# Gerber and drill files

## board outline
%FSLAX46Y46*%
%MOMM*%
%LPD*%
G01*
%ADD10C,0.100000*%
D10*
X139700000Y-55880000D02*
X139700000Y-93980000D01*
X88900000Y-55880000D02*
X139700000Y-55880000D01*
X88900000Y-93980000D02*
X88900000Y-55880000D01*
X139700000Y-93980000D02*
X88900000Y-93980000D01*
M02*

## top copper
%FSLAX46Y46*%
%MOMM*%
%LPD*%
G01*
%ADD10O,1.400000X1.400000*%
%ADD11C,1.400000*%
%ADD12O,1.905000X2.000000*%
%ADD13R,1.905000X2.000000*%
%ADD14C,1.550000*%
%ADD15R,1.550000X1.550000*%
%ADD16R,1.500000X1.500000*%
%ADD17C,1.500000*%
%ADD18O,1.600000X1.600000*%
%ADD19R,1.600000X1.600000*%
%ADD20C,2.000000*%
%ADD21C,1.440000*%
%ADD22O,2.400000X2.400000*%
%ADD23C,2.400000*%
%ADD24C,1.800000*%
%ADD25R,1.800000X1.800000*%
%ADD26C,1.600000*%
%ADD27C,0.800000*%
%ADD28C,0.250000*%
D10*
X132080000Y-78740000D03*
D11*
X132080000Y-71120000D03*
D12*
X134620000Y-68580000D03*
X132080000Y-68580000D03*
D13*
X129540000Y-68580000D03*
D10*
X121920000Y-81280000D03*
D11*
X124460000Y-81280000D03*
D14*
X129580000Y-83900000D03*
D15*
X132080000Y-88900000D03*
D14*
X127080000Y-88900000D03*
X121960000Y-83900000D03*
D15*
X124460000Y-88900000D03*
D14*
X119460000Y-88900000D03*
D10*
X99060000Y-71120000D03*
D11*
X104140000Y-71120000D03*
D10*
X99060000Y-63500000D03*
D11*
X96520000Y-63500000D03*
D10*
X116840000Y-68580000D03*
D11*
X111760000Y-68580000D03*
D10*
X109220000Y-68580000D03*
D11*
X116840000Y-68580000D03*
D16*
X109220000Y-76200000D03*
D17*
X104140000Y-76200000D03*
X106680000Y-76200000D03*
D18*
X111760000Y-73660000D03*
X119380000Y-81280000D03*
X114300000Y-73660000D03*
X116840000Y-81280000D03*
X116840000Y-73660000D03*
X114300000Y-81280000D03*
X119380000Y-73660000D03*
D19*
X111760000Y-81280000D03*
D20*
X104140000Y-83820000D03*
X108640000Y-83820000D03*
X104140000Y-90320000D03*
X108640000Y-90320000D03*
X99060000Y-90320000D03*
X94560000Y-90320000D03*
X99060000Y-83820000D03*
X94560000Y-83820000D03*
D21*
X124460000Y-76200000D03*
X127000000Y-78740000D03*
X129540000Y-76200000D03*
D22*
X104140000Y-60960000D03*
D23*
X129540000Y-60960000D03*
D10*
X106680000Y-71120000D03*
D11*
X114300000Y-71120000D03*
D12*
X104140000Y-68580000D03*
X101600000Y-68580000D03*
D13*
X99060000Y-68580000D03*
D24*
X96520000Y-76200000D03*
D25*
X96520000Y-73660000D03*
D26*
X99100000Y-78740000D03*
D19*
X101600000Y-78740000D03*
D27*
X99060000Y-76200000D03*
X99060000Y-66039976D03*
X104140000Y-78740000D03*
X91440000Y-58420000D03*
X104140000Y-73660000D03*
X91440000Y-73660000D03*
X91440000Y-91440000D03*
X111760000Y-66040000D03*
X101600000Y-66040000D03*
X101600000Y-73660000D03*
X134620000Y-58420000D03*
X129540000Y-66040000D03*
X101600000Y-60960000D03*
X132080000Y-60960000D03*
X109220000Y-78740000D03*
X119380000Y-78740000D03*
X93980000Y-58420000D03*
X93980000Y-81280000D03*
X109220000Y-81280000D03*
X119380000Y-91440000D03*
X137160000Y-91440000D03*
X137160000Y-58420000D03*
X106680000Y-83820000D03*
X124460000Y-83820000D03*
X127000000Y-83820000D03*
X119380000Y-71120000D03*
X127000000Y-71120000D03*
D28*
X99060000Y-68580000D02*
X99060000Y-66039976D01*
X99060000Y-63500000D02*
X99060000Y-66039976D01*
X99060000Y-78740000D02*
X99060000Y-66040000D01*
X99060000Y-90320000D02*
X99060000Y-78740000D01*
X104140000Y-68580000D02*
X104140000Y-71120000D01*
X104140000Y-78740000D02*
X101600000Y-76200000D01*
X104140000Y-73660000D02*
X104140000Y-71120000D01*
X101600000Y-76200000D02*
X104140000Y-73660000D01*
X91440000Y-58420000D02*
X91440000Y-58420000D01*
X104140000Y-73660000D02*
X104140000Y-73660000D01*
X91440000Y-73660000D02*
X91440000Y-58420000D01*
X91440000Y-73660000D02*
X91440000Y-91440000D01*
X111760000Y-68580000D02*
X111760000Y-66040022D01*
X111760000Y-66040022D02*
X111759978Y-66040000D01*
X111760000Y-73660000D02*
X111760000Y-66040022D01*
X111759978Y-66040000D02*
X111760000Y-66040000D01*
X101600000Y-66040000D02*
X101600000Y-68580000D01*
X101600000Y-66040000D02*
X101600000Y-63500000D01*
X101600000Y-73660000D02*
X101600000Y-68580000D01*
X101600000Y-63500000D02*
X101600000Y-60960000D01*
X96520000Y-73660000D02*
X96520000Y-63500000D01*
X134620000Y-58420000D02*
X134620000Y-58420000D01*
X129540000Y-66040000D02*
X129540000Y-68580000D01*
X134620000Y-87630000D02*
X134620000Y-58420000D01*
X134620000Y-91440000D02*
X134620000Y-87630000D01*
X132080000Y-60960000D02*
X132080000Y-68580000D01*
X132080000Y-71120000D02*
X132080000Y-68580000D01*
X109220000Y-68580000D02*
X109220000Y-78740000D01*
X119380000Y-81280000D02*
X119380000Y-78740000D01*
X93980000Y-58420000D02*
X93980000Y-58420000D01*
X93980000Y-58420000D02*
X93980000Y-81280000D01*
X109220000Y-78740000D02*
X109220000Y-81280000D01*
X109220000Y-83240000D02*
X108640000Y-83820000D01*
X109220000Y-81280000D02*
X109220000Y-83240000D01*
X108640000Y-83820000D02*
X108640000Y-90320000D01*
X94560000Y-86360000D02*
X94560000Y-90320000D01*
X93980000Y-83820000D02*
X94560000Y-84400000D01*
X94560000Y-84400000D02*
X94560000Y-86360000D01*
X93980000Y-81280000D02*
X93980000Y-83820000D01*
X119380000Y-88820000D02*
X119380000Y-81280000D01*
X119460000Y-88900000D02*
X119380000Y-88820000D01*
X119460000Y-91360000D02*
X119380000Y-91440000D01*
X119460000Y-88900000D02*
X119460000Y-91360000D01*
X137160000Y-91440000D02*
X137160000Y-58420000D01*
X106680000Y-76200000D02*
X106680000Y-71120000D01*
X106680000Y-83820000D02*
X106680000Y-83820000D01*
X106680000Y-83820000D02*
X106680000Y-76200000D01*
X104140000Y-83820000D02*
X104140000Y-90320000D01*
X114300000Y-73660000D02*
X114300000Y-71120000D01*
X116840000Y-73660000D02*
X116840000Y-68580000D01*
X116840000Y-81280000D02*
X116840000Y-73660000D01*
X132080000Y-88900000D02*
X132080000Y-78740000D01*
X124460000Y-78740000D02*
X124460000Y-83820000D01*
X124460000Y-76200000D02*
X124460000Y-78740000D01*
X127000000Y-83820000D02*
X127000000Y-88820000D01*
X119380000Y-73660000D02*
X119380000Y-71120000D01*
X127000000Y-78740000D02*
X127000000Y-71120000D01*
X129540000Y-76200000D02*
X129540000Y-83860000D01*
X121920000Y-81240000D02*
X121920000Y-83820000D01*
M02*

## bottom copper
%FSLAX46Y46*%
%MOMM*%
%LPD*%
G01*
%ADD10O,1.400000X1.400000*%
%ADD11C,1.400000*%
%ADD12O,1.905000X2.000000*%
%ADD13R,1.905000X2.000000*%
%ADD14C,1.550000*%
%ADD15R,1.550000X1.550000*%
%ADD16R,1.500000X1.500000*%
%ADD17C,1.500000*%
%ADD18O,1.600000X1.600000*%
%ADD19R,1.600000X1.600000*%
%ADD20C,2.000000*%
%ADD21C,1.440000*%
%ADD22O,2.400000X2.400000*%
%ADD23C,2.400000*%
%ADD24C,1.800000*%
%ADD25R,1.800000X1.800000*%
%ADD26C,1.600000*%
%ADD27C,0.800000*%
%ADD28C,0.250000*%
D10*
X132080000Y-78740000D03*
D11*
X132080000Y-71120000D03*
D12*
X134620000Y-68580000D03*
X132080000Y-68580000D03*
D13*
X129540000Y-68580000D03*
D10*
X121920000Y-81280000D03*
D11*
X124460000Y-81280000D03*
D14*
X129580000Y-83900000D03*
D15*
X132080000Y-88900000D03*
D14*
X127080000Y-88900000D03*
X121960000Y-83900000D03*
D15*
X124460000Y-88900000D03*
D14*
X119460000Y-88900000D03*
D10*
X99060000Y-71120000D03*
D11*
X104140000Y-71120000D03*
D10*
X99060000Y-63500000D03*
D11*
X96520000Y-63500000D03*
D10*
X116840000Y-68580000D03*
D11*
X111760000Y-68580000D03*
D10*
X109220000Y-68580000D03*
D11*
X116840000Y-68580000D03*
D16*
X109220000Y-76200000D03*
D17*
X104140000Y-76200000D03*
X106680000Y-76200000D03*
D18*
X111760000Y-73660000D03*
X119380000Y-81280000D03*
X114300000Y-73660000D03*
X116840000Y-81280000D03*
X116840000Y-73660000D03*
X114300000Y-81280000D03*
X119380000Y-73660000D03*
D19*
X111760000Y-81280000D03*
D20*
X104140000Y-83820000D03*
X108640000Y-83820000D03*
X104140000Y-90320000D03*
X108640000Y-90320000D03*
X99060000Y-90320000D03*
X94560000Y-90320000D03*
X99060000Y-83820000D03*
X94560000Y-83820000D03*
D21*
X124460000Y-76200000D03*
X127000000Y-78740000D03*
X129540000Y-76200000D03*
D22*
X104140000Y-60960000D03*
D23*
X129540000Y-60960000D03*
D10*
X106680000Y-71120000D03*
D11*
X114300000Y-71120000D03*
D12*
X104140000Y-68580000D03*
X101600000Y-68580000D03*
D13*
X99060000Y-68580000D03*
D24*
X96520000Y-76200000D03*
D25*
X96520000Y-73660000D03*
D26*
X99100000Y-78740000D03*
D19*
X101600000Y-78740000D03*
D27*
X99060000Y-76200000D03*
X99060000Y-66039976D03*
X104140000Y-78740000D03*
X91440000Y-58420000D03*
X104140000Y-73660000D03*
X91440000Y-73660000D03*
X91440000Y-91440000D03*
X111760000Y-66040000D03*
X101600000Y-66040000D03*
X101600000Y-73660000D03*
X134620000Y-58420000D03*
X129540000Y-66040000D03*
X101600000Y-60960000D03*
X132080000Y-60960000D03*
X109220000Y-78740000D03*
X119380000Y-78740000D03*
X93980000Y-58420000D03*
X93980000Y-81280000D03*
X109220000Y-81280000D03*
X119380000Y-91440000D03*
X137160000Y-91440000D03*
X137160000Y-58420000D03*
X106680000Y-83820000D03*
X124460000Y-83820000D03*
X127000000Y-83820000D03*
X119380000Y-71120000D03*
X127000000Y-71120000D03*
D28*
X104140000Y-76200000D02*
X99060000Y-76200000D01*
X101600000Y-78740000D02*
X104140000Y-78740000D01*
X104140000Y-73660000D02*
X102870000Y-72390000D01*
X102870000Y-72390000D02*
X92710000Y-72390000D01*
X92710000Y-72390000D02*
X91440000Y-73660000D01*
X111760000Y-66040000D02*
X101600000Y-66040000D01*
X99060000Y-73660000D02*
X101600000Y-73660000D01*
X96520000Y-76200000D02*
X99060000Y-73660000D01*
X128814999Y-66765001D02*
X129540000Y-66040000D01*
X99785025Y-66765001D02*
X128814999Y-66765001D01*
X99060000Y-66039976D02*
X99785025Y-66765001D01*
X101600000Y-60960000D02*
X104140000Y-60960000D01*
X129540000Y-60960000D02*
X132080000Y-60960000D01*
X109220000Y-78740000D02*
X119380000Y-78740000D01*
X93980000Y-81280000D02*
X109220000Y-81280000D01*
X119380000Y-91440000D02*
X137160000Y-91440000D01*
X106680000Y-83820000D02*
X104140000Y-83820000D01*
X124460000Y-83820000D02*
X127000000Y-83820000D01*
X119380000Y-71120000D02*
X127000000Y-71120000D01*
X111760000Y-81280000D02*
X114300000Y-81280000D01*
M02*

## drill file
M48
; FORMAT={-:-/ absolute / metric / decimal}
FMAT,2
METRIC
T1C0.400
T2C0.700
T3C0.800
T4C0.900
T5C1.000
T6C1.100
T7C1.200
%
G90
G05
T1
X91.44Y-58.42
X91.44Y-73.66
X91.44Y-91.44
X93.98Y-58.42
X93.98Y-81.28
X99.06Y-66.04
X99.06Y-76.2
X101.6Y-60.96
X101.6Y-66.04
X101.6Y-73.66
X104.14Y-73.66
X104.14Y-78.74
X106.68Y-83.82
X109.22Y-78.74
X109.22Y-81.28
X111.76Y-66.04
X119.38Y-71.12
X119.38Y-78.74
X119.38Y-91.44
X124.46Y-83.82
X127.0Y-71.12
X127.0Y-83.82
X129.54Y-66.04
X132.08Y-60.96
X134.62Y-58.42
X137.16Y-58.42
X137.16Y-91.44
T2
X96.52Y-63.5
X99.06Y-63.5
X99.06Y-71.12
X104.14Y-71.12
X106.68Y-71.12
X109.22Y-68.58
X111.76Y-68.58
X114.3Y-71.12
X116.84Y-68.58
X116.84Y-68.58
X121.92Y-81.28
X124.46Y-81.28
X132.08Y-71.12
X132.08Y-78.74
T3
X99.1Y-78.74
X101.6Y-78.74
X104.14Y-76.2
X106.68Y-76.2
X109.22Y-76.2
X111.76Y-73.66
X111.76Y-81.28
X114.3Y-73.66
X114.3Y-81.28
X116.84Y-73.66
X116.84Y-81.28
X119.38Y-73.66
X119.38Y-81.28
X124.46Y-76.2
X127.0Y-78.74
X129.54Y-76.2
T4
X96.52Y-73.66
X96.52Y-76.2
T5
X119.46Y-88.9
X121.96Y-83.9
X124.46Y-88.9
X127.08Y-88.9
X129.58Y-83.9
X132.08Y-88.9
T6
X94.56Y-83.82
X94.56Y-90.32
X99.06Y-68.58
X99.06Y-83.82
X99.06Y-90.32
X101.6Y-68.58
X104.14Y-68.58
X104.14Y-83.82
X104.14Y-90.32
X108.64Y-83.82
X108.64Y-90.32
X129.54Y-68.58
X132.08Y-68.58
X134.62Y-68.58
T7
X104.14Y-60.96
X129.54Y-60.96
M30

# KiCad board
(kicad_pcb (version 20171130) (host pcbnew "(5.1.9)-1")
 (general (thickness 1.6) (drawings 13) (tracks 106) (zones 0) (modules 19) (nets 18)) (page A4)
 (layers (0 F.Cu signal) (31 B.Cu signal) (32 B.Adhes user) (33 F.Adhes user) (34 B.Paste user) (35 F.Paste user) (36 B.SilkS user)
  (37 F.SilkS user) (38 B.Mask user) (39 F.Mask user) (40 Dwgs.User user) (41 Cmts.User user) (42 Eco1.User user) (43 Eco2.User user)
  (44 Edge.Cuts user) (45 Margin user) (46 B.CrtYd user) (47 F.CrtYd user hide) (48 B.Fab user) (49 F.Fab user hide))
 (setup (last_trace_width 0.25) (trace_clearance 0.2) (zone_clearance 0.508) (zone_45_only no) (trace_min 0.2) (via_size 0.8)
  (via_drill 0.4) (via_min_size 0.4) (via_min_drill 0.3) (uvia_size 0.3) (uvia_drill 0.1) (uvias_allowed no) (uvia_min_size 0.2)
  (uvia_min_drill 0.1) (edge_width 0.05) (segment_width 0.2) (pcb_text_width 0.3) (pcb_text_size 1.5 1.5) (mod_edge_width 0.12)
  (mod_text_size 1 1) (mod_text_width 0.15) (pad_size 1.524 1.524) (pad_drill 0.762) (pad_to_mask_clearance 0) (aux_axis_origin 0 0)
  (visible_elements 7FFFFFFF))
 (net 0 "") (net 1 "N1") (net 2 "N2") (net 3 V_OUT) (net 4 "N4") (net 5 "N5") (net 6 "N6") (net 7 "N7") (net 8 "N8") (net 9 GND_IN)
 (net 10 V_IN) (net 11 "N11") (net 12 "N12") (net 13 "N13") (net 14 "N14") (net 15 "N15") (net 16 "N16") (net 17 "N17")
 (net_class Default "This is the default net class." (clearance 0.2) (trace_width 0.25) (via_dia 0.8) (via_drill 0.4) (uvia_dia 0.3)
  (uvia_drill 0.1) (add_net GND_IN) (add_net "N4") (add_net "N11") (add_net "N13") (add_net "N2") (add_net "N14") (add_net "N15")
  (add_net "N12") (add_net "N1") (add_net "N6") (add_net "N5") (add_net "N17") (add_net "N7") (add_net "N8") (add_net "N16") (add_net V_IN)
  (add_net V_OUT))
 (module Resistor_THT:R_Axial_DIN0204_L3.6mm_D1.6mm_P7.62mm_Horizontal (layer F.Cu) (at 132.08 71.12 270)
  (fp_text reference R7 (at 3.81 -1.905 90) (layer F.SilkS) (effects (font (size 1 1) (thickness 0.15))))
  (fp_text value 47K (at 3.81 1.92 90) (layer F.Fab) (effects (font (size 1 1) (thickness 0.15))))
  (pad 2 thru_hole oval (at 7.62 0 270) (size 1.4 1.4) (drill 0.7) (layers *.Cu *.Mask) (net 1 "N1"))
  (pad 1 thru_hole circle (at 0 0 270) (size 1.4 1.4) (drill 0.7) (layers *.Cu *.Mask) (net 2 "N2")))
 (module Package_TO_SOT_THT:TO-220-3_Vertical (layer F.Cu) (at 129.54 68.58)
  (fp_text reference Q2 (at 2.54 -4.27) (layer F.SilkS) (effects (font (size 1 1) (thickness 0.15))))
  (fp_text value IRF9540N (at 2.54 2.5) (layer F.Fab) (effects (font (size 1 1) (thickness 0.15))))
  (pad 3 thru_hole oval (at 5.08 0) (size 1.905 2) (drill 1.1) (layers *.Cu *.Mask) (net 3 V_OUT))
  (pad 2 thru_hole oval (at 2.54 0) (size 1.905 2) (drill 1.1) (layers *.Cu *.Mask) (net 2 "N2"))
  (pad 1 thru_hole rect (at 0 0) (size 1.905 2) (drill 1.1) (layers *.Cu *.Mask) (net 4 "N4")))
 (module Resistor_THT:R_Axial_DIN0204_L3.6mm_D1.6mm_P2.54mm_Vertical (layer F.Cu) (at 124.46 81.28 180)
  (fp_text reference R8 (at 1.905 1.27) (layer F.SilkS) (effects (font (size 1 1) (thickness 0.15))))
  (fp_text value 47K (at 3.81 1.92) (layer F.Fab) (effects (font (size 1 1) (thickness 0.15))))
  (pad 2 thru_hole oval (at 2.54 0 180) (size 1.4 1.4) (drill 0.7) (layers *.Cu *.Mask) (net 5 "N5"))
  (pad 1 thru_hole circle (at 0 0 180) (size 1.4 1.4) (drill 0.7) (layers *.Cu *.Mask) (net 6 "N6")))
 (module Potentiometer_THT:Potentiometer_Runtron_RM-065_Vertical (layer F.Cu) (at 132.08 88.9 180)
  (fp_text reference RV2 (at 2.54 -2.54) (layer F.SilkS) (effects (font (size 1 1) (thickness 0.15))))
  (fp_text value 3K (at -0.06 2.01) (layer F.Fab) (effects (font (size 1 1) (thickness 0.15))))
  (pad 2 thru_hole circle (at 2.5 5 180) (size 1.55 1.55) (drill 1) (layers *.Cu *.Mask) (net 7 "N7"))
  (pad 1 thru_hole rect (at 0 0 180) (size 1.55 1.55) (drill 1) (layers *.Cu *.Mask) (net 1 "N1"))
  (pad 3 thru_hole circle (at 5 0 180) (size 1.55 1.55) (drill 1) (layers *.Cu *.Mask) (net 6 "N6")))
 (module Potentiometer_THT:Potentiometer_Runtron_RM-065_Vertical (layer F.Cu) (at 124.46 88.9 180)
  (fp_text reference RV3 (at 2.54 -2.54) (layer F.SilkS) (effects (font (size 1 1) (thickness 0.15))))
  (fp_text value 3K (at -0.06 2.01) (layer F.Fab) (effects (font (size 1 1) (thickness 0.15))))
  (pad 2 thru_hole circle (at 2.5 5 180) (size 1.55 1.55) (drill 1) (layers *.Cu *.Mask) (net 5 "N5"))
  (pad 1 thru_hole rect (at 0 0 180) (size 1.55 1.55) (drill 1) (layers *.Cu *.Mask) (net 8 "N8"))
  (pad 3 thru_hole circle (at 5 0 180) (size 1.55 1.55) (drill 1) (layers *.Cu *.Mask) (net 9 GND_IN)))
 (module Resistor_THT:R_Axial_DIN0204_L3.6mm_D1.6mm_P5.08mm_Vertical (layer F.Cu) (at 104.14 71.12 180)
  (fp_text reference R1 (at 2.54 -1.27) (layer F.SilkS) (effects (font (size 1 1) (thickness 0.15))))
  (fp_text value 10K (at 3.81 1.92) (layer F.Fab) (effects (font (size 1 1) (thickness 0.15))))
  (pad 2 thru_hole oval (at 5.08 0 180) (size 1.4 1.4) (drill 0.7) (layers *.Cu *.Mask) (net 4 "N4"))
  (pad 1 thru_hole circle (at 0 0 180) (size 1.4 1.4) (drill 0.7) (layers *.Cu *.Mask) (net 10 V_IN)))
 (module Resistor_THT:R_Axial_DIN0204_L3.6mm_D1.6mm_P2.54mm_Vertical (layer F.Cu) (at 96.52 63.5)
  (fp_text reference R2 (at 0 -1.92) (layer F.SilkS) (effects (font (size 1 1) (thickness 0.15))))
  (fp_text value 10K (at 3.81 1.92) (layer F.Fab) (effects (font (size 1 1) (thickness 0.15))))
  (pad 2 thru_hole oval (at 2.54 0) (size 1.4 1.4) (drill 0.7) (layers *.Cu *.Mask) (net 4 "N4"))
  (pad 1 thru_hole circle (at 0 0) (size 1.4 1.4) (drill 0.7) (layers *.Cu *.Mask) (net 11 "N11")))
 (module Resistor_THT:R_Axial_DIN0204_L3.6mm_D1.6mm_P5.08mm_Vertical (layer F.Cu) (at 111.76 68.58)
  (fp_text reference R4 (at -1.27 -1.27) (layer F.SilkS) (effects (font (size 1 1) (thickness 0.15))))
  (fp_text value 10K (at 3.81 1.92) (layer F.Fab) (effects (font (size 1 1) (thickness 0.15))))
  (pad 2 thru_hole oval (at 5.08 0) (size 1.4 1.4) (drill 0.7) (layers *.Cu *.Mask) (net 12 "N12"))
  (pad 1 thru_hole circle (at 0 0) (size 1.4 1.4) (drill 0.7) (layers *.Cu *.Mask) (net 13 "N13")))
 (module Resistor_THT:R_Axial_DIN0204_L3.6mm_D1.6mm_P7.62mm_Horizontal (layer F.Cu) (at 116.84 68.58 180)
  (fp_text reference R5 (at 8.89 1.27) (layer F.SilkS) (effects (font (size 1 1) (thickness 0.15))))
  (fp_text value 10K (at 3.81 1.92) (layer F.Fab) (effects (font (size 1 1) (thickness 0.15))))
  (pad 2 thru_hole oval (at 7.62 0 180) (size 1.4 1.4) (drill 0.7) (layers *.Cu *.Mask) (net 9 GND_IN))
  (pad 1 thru_hole circle (at 0 0 180) (size 1.4 1.4) (drill 0.7) (layers *.Cu *.Mask) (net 12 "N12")))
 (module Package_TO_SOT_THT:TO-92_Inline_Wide (layer F.Cu) (at 109.22 76.2 180)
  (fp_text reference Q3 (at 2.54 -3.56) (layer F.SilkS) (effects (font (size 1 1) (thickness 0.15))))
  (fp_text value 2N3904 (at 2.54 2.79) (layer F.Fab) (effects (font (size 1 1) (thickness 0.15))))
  (pad 1 thru_hole rect (at 0 0 180) (size 1.5 1.5) (drill 0.8) (layers *.Cu *.Mask) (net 9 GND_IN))
  (pad 3 thru_hole circle (at 5.08 0 180) (size 1.5 1.5) (drill 0.8) (layers *.Cu *.Mask) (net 4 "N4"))
  (pad 2 thru_hole circle (at 2.54 0 180) (size 1.5 1.5) (drill 0.8) (layers *.Cu *.Mask) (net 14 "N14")))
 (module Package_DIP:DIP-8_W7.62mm (layer F.Cu) (at 111.76 81.28 90)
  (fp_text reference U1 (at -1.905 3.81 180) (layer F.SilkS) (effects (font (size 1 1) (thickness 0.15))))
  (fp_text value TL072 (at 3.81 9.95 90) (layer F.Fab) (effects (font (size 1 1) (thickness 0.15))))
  (pad 8 thru_hole oval (at 7.62 0 90) (size 1.6 1.6) (drill 0.8) (layers *.Cu *.Mask) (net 13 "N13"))
  (pad 4 thru_hole oval (at 0 7.62 90) (size 1.6 1.6) (drill 0.8) (layers *.Cu *.Mask) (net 9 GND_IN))
  (pad 7 thru_hole oval (at 7.62 2.54 90) (size 1.6 1.6) (drill 0.8) (layers *.Cu *.Mask) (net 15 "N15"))
  (pad 3 thru_hole oval (at 0 5.08 90) (size 1.6 1.6) (drill 0.8) (layers *.Cu *.Mask) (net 12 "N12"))
  (pad 6 thru_hole oval (at 7.62 5.08 90) (size 1.6 1.6) (drill 0.8) (layers *.Cu *.Mask) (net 12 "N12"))
  (pad 2 thru_hole oval (at 0 2.54 90) (size 1.6 1.6) (drill 0.8) (layers *.Cu *.Mask) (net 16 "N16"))
  (pad 5 thru_hole oval (at 7.62 7.62 90) (size 1.6 1.6) (drill 0.8) (layers *.Cu *.Mask) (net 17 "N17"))
  (pad 1 thru_hole rect (at 0 0 90) (size 1.6 1.6) (drill 0.8) (layers *.Cu *.Mask) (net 16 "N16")))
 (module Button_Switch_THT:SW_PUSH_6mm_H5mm (layer F.Cu) (at 104.14 90.32 90)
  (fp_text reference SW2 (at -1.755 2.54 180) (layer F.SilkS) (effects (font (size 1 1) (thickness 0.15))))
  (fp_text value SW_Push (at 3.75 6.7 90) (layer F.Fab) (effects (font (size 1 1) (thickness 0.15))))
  (pad 1 thru_hole circle (at 6.5 0 180) (size 2 2) (drill 1.1) (layers *.Cu *.Mask) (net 14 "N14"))
  (pad 2 thru_hole circle (at 6.5 4.5 180) (size 2 2) (drill 1.1) (layers *.Cu *.Mask) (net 9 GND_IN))
  (pad 1 thru_hole circle (at 0 0 180) (size 2 2) (drill 1.1) (layers *.Cu *.Mask) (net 14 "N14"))
  (pad 2 thru_hole circle (at 0 4.5 180) (size 2 2) (drill 1.1) (layers *.Cu *.Mask) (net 9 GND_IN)))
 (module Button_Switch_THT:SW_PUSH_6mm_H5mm (layer F.Cu) (at 99.06 83.82 270)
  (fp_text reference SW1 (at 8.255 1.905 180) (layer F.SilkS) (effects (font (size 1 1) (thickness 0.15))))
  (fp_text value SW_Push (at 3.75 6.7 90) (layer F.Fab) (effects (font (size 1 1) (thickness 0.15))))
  (pad 1 thru_hole circle (at 6.5 0) (size 2 2) (drill 1.1) (layers *.Cu *.Mask) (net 4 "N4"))
  (pad 2 thru_hole circle (at 6.5 4.5) (size 2 2) (drill 1.1) (layers *.Cu *.Mask) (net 9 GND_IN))
  (pad 1 thru_hole circle (at 0 0) (size 2 2) (drill 1.1) (layers *.Cu *.Mask) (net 4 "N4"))
  (pad 2 thru_hole circle (at 0 4.5) (size 2 2) (drill 1.1) (layers *.Cu *.Mask) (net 9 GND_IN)))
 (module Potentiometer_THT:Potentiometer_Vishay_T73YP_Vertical (layer F.Cu) (at 124.46 76.2 270)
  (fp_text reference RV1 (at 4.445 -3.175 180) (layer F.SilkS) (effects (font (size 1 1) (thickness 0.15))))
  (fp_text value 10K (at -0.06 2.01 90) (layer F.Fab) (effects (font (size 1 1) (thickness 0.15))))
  (pad 1 thru_hole circle (at 0 0 270) (size 1.44 1.44) (drill 0.8) (layers *.Cu *.Mask) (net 6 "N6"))
  (pad 2 thru_hole circle (at 2.54 -2.54 270) (size 1.44 1.44) (drill 0.8) (layers *.Cu *.Mask) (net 17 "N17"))
  (pad 3 thru_hole circle (at 0 -5.08 270) (size 1.44 1.44) (drill 0.8) (layers *.Cu *.Mask) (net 7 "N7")))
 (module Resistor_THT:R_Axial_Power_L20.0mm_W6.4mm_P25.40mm (layer F.Cu) (at 129.54 60.96 180)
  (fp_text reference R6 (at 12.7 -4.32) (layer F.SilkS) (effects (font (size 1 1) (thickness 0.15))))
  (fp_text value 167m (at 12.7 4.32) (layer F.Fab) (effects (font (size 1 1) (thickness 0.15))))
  (pad 2 thru_hole oval (at 25.4 0 180) (size 2.4 2.4) (drill 1.2) (layers *.Cu *.Mask) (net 13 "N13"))
  (pad 1 thru_hole circle (at 0 0 180) (size 2.4 2.4) (drill 1.2) (layers *.Cu *.Mask) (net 2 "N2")))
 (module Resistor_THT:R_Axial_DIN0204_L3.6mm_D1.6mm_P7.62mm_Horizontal (layer F.Cu) (at 114.3 71.12 180)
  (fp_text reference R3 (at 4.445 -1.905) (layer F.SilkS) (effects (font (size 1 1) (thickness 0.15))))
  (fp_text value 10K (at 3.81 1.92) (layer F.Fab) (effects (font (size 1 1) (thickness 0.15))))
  (pad 2 thru_hole oval (at 7.62 0 180) (size 1.4 1.4) (drill 0.7) (layers *.Cu *.Mask) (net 14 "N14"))
  (pad 1 thru_hole circle (at 0 0 180) (size 1.4 1.4) (drill 0.7) (layers *.Cu *.Mask) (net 15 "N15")))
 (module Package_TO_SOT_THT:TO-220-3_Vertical (layer F.Cu) (at 99.06 68.58)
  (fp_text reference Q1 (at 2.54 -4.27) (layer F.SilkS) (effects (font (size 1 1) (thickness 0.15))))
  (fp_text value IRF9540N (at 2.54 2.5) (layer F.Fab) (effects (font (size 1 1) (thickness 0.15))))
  (pad 3 thru_hole oval (at 5.08 0) (size 1.905 2) (drill 1.1) (layers *.Cu *.Mask) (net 10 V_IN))
  (pad 2 thru_hole oval (at 2.54 0) (size 1.905 2) (drill 1.1) (layers *.Cu *.Mask) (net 13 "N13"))
  (pad 1 thru_hole rect (at 0 0) (size 1.905 2) (drill 1.1) (layers *.Cu *.Mask) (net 4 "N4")))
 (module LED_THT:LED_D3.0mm (layer F.Cu) (at 96.52 73.66 270)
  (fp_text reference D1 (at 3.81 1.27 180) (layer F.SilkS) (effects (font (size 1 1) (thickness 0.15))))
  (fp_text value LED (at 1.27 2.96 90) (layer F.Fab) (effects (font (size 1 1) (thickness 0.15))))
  (pad 2 thru_hole circle (at 2.54 0 270) (size 1.8 1.8) (drill 0.9) (layers *.Cu *.Mask) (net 13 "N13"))
  (pad 1 thru_hole rect (at 0 0 270) (size 1.8 1.8) (drill 0.9) (layers *.Cu *.Mask) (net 11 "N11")))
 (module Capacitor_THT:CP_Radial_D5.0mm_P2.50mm (layer F.Cu) (at 101.6 78.74 180)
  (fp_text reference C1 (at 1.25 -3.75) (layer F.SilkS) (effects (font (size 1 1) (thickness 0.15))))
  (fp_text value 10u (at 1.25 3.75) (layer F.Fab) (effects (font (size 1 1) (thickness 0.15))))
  (pad 2 thru_hole circle (at 2.5 0 180) (size 1.6 1.6) (drill 0.8) (layers *.Cu *.Mask) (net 4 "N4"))
  (pad 1 thru_hole rect (at 0 0 180) (size 1.6 1.6) (drill 0.8) (layers *.Cu *.Mask) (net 10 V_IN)))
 (gr_line (start 139.7 55.88) (end 139.7 93.98) (layer Edge.Cuts) (width 0.1))
 (gr_line (start 88.9 55.88) (end 139.7 55.88) (layer Edge.Cuts) (width 0.1))
 (gr_line (start 88.9 93.98) (end 88.9 55.88) (layer Edge.Cuts) (width 0.1))
 (gr_line (start 139.7 93.98) (end 88.9 93.98) (layer Edge.Cuts) (width 0.1))
 (via (at 99.06 76.2) (size 0.8) (drill 0.4) (layers F.Cu B.Cu) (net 4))
 (segment (start 104.14 76.2) (end 99.06 76.2) (width 0.25) (layer B.Cu) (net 4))
 (via (at 99.06 66.039976) (size 0.8) (drill 0.4) (layers F.Cu B.Cu) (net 4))
 (segment (start 99.06 68.58) (end 99.06 66.039976) (width 0.25) (layer F.Cu) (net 4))
 (segment (start 99.06 63.5) (end 99.06 66.039976) (width 0.25) (layer F.Cu) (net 4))
 (segment (start 99.06 78.74) (end 99.06 66.04) (width 0.25) (layer F.Cu) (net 4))
 (segment (start 99.06 90.32) (end 99.06 78.74) (width 0.25) (layer F.Cu) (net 4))
 (segment (start 104.14 68.58) (end 104.14 71.12) (width 0.25) (layer F.Cu) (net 10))
 (via (at 104.14 78.74) (size 0.8) (drill 0.4) (layers F.Cu B.Cu) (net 10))
 (segment (start 101.6 78.74) (end 104.14 78.74) (width 0.25) (layer B.Cu) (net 10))
 (segment (start 104.14 78.74) (end 101.6 76.2) (width 0.25) (layer F.Cu) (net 10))
 (segment (start 104.14 73.66) (end 104.14 71.12) (width 0.25) (layer F.Cu) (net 10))
 (segment (start 101.6 76.2) (end 104.14 73.66) (width 0.25) (layer F.Cu) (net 10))
 (segment (start 91.44 58.42) (end 91.44 58.42) (width 0.25) (layer F.Cu) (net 10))
 (via (at 91.44 58.42) (size 0.8) (drill 0.4) (layers F.Cu B.Cu) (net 10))
 (segment (start 104.14 73.66) (end 104.14 73.66) (width 0.25) (layer F.Cu) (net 10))
 (via (at 104.14 73.66) (size 0.8) (drill 0.4) (layers F.Cu B.Cu) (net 10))
 (segment (start 104.14 73.66) (end 102.87 72.39) (width 0.25) (layer B.Cu) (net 10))
 (segment (start 102.87 72.39) (end 92.71 72.39) (width 0.25) (layer B.Cu) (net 10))
 (via (at 91.44 73.66) (size 0.8) (drill 0.4) (layers F.Cu B.Cu) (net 10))
 (segment (start 92.71 72.39) (end 91.44 73.66) (width 0.25) (layer B.Cu) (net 10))
 (segment (start 91.44 73.66) (end 91.44 58.42) (width 0.25) (layer F.Cu) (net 10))
 (via (at 91.44 91.44) (size 0.8) (drill 0.4) (layers F.Cu B.Cu) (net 10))
 (segment (start 91.44 73.66) (end 91.44 91.44) (width 0.25) (layer F.Cu) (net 10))
 (segment (start 111.76 68.58) (end 111.76 66.040022) (width 0.25) (layer F.Cu) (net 13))
 (segment (start 111.76 66.040022) (end 111.759978 66.04) (width 0.25) (layer F.Cu) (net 13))
 (segment (start 111.76 73.66) (end 111.76 66.040022) (width 0.25) (layer F.Cu) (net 13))
 (via (at 111.76 66.04) (size 0.8) (drill 0.4) (layers F.Cu B.Cu) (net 13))
 (segment (start 111.759978 66.04) (end 111.76 66.04) (width 0.25) (layer F.Cu) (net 13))
 (via (at 101.6 66.04) (size 0.8) (drill 0.4) (layers F.Cu B.Cu) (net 13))
 (segment (start 111.76 66.04) (end 101.6 66.04) (width 0.25) (layer B.Cu) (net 13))
 (segment (start 101.6 66.04) (end 101.6 68.58) (width 0.25) (layer F.Cu) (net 13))
 (segment (start 101.6 66.04) (end 101.6 63.5) (width 0.25) (layer F.Cu) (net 13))
 (via (at 101.6 73.66) (size 0.8) (drill 0.4) (layers F.Cu B.Cu) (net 13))
 (segment (start 101.6 73.66) (end 101.6 68.58) (width 0.25) (layer F.Cu) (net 13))
 (segment (start 101.6 63.5) (end 101.6 60.96) (width 0.25) (layer F.Cu) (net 13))
 (segment (start 99.06 73.66) (end 101.6 73.66) (width 0.25) (layer B.Cu) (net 13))
 (segment (start 96.52 76.2) (end 99.06 73.66) (width 0.25) (layer B.Cu) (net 13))
 (segment (start 96.52 73.66) (end 96.52 63.5) (width 0.25) (layer F.Cu) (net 11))
 (segment (start 134.62 58.42) (end 134.62 58.42) (width 0.25) (layer F.Cu) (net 3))
 (via (at 134.62 58.42) (size 0.8) (drill 0.4) (layers F.Cu B.Cu) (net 3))
 (segment (start 128.814999 66.765001) (end 129.54 66.04) (width 0.25) (layer B.Cu) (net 4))
 (segment (start 99.785025 66.765001) (end 128.814999 66.765001) (width 0.25) (layer B.Cu) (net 4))
 (segment (start 99.06 66.039976) (end 99.785025 66.765001) (width 0.25) (layer B.Cu) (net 4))
 (via (at 129.54 66.04) (size 0.8) (drill 0.4) (layers F.Cu B.Cu) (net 4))
 (segment (start 129.54 66.04) (end 129.54 68.58) (width 0.25) (layer F.Cu) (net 4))
 (via (at 101.6 60.96) (size 0.8) (drill 0.4) (layers F.Cu B.Cu) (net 13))
 (segment (start 101.6 60.96) (end 104.14 60.96) (width 0.25) (layer B.Cu) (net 13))
 (segment (start 134.62 87.63) (end 134.62 58.42) (width 0.25) (layer F.Cu) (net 3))
 (segment (start 134.62 91.44) (end 134.62 87.63) (width 0.25) (layer F.Cu) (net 3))
 (via (at 132.08 60.96) (size 0.8) (drill 0.4) (layers F.Cu B.Cu) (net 2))
 (segment (start 129.54 60.96) (end 132.08 60.96) (width 0.25) (layer B.Cu) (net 2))
 (segment (start 132.08 60.96) (end 132.08 68.58) (width 0.25) (layer F.Cu) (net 2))
 (segment (start 132.08 71.12) (end 132.08 68.58) (width 0.25) (layer F.Cu) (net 2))
 (via (at 109.22 78.74) (size 0.8) (drill 0.4) (layers F.Cu B.Cu) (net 9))
 (segment (start 109.22 68.58) (end 109.22 78.74) (width 0.25) (layer F.Cu) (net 9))
 (segment (start 109.22 78.74) (end 119.38 78.74) (width 0.25) (layer B.Cu) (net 9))
 (via (at 119.38 78.74) (size 0.8) (drill 0.4) (layers F.Cu B.Cu) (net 9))
 (segment (start 119.38 81.28) (end 119.38 78.74) (width 0.25) (layer F.Cu) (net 9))
 (segment (start 93.98 58.42) (end 93.98 58.42) (width 0.25) (layer F.Cu) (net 9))
 (via (at 93.98 58.42) (size 0.8) (drill 0.4) (layers F.Cu B.Cu) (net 9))
 (segment (start 93.98 58.42) (end 93.98 81.28) (width 0.25) (layer F.Cu) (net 9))
 (via (at 93.98 81.28) (size 0.8) (drill 0.4) (layers F.Cu B.Cu) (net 9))
 (segment (start 93.98 81.28) (end 109.22 81.28) (width 0.25) (layer B.Cu) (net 9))
 (via (at 109.22 81.28) (size 0.8) (drill 0.4) (layers F.Cu B.Cu) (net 9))
 (segment (start 109.22 78.74) (end 109.22 81.28) (width 0.25) (layer F.Cu) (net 9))
 (segment (start 109.22 83.24) (end 108.64 83.82) (width 0.25) (layer F.Cu) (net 9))
 (segment (start 109.22 81.28) (end 109.22 83.24) (width 0.25) (layer F.Cu) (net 9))
 (segment (start 108.64 83.82) (end 108.64 90.32) (width 0.25) (layer F.Cu) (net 9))
 (segment (start 94.56 86.36) (end 94.56 90.32) (width 0.25) (layer F.Cu) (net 9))
 (segment (start 93.98 83.82) (end 94.56 84.4) (width 0.25) (layer F.Cu) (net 9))
 (segment (start 94.56 84.4) (end 94.56 86.36) (width 0.25) (layer F.Cu) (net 9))
 (segment (start 93.98 81.28) (end 93.98 83.82) (width 0.25) (layer F.Cu) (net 9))
 (segment (start 119.38 88.82) (end 119.38 81.28) (width 0.25) (layer F.Cu) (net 9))
 (segment (start 119.46 88.9) (end 119.38 88.82) (width 0.25) (layer F.Cu) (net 9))
 (via (at 119.38 91.44) (size 0.8) (drill 0.4) (layers F.Cu B.Cu) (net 9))
 (segment (start 119.46 91.36) (end 119.38 91.44) (width 0.25) (layer F.Cu) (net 9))
 (segment (start 119.46 88.9) (end 119.46 91.36) (width 0.25) (layer F.Cu) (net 9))
 (segment (start 119.38 91.44) (end 137.16 91.44) (width 0.25) (layer B.Cu) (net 9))
 (via (at 137.16 91.44) (size 0.8) (drill 0.4) (layers F.Cu B.Cu) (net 9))
 (via (at 137.16 58.42) (size 0.8) (drill 0.4) (layers F.Cu B.Cu) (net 9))
 (segment (start 137.16 91.44) (end 137.16 58.42) (width 0.25) (layer F.Cu) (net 9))
 (segment (start 106.68 76.2) (end 106.68 71.12) (width 0.25) (layer F.Cu) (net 14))
 (segment (start 106.68 83.82) (end 106.68 83.82) (width 0.25) (layer F.Cu) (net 14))
 (segment (start 106.68 83.82) (end 106.68 76.2) (width 0.25) (layer F.Cu) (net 14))
 (via (at 106.68 83.82) (size 0.8) (drill 0.4) (layers F.Cu B.Cu) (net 14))
 (segment (start 106.68 83.82) (end 104.14 83.82) (width 0.25) (layer B.Cu) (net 14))
 (segment (start 104.14 83.82) (end 104.14 90.32) (width 0.25) (layer F.Cu) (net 14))
 (segment (start 114.3 73.66) (end 114.3 71.12) (width 0.25) (layer F.Cu) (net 15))
 (segment (start 116.84 73.66) (end 116.84 68.58) (width 0.25) (layer F.Cu) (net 12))
 (segment (start 116.84 81.28) (end 116.84 73.66) (width 0.25) (layer F.Cu) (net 12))
 (segment (start 132.08 88.9) (end 132.08 78.74) (width 0.25) (layer F.Cu) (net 1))
 (segment (start 124.46 78.74) (end 124.46 83.82) (width 0.25) (layer F.Cu) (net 6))
 (via (at 124.46 83.82) (size 0.8) (drill 0.4) (layers F.Cu B.Cu) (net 6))
 (segment (start 124.46 76.2) (end 124.46 78.74) (width 0.25) (layer F.Cu) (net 6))
 (via (at 127 83.82) (size 0.8) (drill 0.4) (layers F.Cu B.Cu) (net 6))
 (segment (start 124.46 83.82) (end 127 83.82) (width 0.25) (layer B.Cu) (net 6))
 (segment (start 127 83.82) (end 127 88.82) (width 0.25) (layer F.Cu) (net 6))
 (via (at 119.38 71.12) (size 0.8) (drill 0.4) (layers F.Cu B.Cu) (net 17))
 (segment (start 119.38 73.66) (end 119.38 71.12) (width 0.25) (layer F.Cu) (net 17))
 (segment (start 119.38 71.12) (end 127 71.12) (width 0.25) (layer B.Cu) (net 17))
 (segment (start 127 78.74) (end 127 71.12) (width 0.25) (layer F.Cu) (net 17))
 (via (at 127 71.12) (size 0.8) (drill 0.4) (layers F.Cu B.Cu) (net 17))
 (segment (start 111.76 81.28) (end 114.3 81.28) (width 0.25) (layer B.Cu) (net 16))
 (segment (start 129.54 76.2) (end 129.54 83.86) (width 0.25) (layer F.Cu) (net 7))
 (segment (start 121.92 81.24) (end 121.92 83.82) (width 0.25) (layer F.Cu) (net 5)))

